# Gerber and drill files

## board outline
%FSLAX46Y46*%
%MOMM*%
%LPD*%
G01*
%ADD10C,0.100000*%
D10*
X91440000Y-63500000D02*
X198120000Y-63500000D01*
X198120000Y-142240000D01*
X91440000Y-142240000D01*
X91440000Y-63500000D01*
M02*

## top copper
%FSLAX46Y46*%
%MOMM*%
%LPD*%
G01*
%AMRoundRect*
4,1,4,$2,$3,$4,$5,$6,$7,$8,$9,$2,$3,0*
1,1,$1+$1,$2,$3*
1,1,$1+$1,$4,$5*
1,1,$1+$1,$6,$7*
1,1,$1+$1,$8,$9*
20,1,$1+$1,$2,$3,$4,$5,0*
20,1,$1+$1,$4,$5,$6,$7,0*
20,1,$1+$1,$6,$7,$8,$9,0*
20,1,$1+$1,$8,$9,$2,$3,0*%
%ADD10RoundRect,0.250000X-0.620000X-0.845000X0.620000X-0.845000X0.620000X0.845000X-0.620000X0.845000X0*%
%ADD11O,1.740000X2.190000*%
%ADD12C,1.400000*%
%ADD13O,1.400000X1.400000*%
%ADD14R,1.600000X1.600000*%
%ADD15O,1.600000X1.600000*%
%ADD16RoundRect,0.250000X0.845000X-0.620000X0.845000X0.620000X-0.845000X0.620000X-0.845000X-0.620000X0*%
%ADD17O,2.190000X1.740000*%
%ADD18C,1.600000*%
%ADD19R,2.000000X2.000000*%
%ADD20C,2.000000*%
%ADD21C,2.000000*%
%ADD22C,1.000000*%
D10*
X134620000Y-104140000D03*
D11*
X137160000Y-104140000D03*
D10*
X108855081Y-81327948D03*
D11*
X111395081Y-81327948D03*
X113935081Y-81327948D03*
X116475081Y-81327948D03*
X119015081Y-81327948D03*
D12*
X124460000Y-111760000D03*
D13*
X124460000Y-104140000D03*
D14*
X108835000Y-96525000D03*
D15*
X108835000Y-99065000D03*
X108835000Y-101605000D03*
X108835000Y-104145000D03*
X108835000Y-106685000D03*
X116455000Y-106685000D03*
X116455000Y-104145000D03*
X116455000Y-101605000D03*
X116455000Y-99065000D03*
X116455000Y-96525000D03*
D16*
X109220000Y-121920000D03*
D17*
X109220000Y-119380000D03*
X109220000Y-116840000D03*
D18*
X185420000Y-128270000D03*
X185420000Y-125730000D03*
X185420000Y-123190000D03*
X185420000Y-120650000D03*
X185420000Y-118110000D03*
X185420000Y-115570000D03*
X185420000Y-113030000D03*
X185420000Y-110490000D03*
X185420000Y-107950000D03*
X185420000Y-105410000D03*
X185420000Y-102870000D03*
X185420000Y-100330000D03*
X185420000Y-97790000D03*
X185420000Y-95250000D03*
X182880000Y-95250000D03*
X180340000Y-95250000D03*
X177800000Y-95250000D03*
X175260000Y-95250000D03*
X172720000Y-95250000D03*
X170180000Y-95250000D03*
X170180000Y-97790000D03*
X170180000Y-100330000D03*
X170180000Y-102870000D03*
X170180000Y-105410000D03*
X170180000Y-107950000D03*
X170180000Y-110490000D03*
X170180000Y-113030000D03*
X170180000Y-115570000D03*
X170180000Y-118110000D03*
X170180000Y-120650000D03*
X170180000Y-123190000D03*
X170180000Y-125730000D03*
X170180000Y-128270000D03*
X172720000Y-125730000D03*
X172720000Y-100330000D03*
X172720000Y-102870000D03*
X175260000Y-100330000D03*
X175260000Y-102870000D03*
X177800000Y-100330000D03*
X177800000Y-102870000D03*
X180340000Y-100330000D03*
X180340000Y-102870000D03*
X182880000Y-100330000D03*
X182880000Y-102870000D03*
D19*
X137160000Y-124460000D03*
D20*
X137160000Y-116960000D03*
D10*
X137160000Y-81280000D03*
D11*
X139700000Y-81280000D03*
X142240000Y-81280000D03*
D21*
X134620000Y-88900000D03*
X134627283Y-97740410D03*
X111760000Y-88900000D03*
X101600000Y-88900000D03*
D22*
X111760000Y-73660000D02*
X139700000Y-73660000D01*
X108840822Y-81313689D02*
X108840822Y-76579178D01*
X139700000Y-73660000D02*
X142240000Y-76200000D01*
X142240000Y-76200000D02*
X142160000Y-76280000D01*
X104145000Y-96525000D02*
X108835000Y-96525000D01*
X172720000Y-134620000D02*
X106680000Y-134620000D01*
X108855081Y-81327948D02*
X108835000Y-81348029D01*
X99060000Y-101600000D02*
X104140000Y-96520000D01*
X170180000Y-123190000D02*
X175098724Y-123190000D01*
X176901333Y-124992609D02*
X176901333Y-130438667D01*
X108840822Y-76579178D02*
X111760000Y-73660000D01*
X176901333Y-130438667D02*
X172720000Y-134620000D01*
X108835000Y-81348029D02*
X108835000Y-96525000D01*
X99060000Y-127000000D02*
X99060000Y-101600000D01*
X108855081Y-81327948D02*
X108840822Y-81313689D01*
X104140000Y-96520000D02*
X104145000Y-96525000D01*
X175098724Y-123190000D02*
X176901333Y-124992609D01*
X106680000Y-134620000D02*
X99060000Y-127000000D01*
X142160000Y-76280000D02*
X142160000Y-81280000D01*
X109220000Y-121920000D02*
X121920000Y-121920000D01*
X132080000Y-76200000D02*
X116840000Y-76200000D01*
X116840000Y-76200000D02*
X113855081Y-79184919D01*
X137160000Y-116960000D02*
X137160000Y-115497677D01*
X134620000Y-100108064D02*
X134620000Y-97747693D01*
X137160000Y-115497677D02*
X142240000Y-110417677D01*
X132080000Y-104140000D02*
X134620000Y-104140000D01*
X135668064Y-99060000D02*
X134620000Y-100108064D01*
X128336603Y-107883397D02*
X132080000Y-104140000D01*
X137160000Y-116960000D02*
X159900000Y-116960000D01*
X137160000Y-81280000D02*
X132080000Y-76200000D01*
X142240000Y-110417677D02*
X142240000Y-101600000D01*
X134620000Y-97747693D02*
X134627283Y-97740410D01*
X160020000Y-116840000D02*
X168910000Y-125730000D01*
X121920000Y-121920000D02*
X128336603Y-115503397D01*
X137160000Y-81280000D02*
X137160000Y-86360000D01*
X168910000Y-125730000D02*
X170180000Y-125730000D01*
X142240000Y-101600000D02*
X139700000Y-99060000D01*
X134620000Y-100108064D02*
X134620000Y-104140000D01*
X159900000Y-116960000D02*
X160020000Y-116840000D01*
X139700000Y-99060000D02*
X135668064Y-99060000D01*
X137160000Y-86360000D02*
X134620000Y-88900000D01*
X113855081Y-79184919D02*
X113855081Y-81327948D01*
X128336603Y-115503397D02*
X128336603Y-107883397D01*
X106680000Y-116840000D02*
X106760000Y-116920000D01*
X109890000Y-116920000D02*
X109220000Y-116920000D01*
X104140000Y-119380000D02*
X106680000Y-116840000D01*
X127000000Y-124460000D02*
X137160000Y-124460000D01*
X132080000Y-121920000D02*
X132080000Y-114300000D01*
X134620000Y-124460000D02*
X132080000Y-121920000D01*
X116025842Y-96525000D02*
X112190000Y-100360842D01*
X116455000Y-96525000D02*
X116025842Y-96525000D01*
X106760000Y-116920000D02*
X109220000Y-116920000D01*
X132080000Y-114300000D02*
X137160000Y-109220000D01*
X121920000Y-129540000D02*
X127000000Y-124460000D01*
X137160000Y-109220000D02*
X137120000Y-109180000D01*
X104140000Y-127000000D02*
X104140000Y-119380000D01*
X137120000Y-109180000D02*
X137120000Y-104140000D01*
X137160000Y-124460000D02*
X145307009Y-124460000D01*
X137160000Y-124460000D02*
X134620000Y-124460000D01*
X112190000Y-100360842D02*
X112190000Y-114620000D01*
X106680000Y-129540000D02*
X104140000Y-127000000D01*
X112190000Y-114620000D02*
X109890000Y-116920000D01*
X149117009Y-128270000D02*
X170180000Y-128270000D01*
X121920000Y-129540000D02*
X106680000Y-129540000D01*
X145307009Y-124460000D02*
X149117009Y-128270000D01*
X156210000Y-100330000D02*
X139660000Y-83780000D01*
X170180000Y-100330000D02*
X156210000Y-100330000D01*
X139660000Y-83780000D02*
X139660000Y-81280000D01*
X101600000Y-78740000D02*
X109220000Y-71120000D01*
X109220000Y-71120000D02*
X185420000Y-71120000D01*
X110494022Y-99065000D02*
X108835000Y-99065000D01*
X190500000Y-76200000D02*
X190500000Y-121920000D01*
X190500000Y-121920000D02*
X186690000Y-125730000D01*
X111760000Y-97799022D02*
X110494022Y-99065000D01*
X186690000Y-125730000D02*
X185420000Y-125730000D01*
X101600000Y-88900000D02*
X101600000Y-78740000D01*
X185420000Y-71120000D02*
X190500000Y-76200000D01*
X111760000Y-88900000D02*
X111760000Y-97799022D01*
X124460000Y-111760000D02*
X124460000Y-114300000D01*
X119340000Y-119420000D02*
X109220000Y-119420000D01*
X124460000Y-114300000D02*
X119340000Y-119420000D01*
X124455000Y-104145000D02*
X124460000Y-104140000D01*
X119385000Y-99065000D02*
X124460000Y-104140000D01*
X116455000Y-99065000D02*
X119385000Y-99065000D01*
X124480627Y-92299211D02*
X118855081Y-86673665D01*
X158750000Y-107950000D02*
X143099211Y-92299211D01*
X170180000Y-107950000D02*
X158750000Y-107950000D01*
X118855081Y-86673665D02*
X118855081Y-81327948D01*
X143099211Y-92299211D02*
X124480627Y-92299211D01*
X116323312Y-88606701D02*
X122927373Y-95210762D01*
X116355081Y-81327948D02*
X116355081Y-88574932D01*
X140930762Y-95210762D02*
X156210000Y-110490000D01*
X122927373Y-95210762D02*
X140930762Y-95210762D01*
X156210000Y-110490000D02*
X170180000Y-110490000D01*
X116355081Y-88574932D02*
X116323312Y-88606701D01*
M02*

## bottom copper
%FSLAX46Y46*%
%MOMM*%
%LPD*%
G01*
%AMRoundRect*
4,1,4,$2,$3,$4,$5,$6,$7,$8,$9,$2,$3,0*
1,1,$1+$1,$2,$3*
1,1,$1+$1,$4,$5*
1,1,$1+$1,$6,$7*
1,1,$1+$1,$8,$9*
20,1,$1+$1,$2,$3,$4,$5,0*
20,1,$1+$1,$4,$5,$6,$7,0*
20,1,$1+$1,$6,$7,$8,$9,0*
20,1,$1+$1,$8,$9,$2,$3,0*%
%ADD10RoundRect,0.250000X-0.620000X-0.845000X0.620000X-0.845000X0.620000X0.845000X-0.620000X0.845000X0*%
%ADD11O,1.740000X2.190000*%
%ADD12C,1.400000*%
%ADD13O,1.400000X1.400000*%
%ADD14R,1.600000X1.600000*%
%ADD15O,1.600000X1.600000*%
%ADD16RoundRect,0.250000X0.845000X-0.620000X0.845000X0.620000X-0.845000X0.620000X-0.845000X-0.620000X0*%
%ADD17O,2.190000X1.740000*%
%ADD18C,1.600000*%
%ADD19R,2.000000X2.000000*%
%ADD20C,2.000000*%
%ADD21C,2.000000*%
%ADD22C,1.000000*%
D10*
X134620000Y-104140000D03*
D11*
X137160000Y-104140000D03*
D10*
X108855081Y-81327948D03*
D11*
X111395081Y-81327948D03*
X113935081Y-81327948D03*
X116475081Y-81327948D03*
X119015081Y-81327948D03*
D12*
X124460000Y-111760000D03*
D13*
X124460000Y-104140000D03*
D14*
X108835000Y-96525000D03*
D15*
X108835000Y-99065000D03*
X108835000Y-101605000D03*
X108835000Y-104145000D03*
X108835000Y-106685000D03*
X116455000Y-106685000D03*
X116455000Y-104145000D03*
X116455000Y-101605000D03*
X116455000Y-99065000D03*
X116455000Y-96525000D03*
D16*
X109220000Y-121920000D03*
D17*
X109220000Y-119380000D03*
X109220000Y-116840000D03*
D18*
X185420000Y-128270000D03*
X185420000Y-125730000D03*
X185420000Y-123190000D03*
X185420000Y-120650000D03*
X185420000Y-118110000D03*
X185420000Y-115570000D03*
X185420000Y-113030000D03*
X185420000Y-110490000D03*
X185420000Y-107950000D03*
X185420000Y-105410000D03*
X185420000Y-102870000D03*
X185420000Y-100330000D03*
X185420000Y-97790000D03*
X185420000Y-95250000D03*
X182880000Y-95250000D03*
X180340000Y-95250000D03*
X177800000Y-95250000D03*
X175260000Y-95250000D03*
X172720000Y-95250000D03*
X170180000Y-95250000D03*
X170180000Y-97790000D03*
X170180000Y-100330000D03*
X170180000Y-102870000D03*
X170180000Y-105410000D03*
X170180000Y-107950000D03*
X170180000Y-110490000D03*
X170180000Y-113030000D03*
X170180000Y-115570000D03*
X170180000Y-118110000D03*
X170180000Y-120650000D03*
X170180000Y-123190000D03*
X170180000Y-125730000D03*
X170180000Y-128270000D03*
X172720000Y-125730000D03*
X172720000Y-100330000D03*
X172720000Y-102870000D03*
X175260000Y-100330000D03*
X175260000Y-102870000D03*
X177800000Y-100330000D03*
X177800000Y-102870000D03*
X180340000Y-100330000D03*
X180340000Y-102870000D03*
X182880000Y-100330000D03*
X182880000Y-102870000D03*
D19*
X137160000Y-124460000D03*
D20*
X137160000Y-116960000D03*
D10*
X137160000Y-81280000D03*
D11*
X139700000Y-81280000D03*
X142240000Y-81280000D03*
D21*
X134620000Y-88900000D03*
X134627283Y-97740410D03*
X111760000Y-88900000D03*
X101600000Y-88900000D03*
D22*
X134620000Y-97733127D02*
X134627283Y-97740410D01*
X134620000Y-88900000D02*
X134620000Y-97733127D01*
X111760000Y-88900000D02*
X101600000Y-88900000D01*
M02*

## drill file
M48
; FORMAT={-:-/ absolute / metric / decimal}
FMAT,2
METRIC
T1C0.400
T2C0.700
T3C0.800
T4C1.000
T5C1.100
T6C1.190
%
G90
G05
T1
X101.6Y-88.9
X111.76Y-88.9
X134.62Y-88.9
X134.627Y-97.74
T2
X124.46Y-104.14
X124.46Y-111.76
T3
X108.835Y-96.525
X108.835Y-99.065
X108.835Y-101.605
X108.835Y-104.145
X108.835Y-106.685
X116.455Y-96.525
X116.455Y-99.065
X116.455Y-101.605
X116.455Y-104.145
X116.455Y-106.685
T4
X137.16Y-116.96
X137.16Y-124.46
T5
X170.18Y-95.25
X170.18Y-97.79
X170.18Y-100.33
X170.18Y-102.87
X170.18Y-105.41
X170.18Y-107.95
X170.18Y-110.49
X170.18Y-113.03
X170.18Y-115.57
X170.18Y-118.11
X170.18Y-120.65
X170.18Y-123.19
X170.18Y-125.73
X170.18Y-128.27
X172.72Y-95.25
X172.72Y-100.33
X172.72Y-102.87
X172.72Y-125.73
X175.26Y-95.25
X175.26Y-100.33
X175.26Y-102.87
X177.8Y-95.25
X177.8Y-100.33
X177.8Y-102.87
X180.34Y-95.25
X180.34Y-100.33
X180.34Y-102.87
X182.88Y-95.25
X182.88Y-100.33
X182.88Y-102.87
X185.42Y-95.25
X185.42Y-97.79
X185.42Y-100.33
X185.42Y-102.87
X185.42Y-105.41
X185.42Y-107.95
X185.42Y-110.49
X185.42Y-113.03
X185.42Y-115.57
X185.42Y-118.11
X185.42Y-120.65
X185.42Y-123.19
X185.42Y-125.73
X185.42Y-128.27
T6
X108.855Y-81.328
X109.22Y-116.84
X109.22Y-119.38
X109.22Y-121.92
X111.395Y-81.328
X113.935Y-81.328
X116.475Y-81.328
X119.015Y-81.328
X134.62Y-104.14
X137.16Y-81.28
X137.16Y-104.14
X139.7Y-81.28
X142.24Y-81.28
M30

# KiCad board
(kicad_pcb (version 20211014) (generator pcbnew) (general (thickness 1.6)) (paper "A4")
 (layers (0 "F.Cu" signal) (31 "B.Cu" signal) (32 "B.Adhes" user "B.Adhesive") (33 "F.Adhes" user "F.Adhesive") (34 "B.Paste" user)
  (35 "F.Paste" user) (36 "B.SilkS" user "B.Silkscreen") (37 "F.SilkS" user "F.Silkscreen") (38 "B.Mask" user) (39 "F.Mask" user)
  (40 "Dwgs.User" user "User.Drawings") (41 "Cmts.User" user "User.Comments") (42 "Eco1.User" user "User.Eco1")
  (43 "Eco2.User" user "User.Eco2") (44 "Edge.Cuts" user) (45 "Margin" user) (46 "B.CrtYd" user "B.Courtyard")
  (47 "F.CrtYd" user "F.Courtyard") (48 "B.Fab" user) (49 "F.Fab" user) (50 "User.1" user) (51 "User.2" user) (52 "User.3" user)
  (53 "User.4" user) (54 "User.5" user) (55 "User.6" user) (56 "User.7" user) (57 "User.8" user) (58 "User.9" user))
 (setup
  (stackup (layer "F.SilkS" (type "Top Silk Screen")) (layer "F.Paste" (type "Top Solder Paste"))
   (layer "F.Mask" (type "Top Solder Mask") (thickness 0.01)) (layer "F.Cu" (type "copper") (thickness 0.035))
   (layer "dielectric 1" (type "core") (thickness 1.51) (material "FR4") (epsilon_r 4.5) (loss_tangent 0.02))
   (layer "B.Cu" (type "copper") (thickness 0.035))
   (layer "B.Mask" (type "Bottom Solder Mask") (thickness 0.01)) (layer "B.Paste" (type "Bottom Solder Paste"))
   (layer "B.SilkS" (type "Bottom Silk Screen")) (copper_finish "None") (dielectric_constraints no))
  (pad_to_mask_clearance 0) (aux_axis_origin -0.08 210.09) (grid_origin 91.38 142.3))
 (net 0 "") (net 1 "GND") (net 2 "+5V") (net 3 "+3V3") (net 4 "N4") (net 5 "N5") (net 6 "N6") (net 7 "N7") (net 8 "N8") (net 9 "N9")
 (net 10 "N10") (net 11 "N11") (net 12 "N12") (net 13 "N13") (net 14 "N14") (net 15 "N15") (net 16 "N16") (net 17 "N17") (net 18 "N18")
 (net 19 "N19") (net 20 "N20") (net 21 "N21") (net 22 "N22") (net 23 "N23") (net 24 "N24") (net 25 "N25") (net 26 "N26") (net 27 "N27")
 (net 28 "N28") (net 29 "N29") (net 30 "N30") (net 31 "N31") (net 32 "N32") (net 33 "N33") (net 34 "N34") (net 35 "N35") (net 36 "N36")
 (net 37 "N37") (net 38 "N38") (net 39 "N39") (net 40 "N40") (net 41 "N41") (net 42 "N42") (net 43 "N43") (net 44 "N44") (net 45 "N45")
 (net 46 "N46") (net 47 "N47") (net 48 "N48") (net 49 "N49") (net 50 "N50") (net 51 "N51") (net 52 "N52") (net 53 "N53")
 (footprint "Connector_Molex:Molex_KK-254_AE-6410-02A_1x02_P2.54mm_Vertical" (layer "F.Cu") (at 134.62 104.14)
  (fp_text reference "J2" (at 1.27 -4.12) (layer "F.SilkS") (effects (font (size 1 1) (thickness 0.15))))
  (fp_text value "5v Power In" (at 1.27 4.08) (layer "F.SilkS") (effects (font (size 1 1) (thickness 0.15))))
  (pad "1" thru_hole roundrect (at 0 0) (size 1.74 2.19) (drill 1.19) (layers *.Cu *.Mask) (roundrect_rratio 0.1436781609) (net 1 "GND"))
  (pad "2" thru_hole oval (at 2.54 0) (size 1.74 2.19) (drill 1.19) (layers *.Cu *.Mask) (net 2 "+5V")))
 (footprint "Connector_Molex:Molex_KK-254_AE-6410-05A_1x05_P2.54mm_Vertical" (layer "F.Cu") (at 108.855081 81.327948)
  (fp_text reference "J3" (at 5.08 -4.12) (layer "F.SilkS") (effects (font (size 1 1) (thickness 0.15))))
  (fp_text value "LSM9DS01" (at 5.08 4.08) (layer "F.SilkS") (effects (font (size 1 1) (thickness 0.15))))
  (pad "1" thru_hole roundrect (at 0 0) (size 1.74 2.19) (drill 1.19) (layers *.Cu *.Mask) (roundrect_rratio 0.1436781609) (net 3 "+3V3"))
  (pad "2" thru_hole oval (at 2.54 0) (size 1.74 2.19) (drill 1.19) (layers *.Cu *.Mask) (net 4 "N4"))
  (pad "3" thru_hole oval (at 5.08 0) (size 1.74 2.19) (drill 1.19) (layers *.Cu *.Mask) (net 1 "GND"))
  (pad "4" thru_hole oval (at 7.62 0) (size 1.74 2.19) (drill 1.19) (layers *.Cu *.Mask) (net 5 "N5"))
  (pad "5" thru_hole oval (at 10.16 0) (size 1.74 2.19) (drill 1.19) (layers *.Cu *.Mask) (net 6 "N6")))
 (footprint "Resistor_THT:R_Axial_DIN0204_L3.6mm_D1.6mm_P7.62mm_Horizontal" (layer "F.Cu") (at 124.46 111.76 90)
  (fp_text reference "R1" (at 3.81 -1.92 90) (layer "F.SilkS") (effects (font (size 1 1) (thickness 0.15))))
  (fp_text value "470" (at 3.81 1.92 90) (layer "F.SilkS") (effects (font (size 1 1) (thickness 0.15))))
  (pad "1" thru_hole circle (at 0 0 90) (size 1.4 1.4) (drill 0.7) (layers *.Cu *.Mask) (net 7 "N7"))
  (pad "2" thru_hole oval (at 7.62 0 90) (size 1.4 1.4) (drill 0.7) (layers *.Cu *.Mask) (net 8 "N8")))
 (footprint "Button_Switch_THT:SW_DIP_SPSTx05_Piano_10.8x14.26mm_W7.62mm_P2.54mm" (layer "F.Cu") (at 108.835 96.525)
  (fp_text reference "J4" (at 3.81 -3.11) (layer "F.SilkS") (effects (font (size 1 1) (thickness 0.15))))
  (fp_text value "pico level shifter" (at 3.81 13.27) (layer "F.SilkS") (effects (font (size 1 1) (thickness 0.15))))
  (pad "1" thru_hole rect (at 0 0) (size 1.6 1.6) (drill 0.8) (layers *.Cu *.Mask) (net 3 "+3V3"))
  (pad "2" thru_hole oval (at 0 2.54) (size 1.6 1.6) (drill 0.8) (layers *.Cu *.Mask) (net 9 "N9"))
  (pad "3" thru_hole oval (at 0 5.08) (size 1.6 1.6) (drill 0.8) (layers *.Cu *.Mask) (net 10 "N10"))
  (pad "4" thru_hole oval (at 0 7.62) (size 1.6 1.6) (drill 0.8) (layers *.Cu *.Mask) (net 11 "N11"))
  (pad "5" thru_hole oval (at 0 10.16) (size 1.6 1.6) (drill 0.8) (layers *.Cu *.Mask) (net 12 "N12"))
  (pad "6" thru_hole oval (at 7.62 10.16) (size 1.6 1.6) (drill 0.8) (layers *.Cu *.Mask) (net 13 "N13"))
  (pad "7" thru_hole oval (at 7.62 7.62) (size 1.6 1.6) (drill 0.8) (layers *.Cu *.Mask) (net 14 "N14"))
  (pad "8" thru_hole oval (at 7.62 5.08) (size 1.6 1.6) (drill 0.8) (layers *.Cu *.Mask) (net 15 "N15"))
  (pad "9" thru_hole oval (at 7.62 2.54) (size 1.6 1.6) (drill 0.8) (layers *.Cu *.Mask) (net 8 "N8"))
  (pad "10" thru_hole oval (at 7.62 0) (size 1.6 1.6) (drill 0.8) (layers *.Cu *.Mask) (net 2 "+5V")))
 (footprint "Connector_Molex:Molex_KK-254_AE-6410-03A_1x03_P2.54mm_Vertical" (layer "F.Cu") (at 109.22 121.92 90)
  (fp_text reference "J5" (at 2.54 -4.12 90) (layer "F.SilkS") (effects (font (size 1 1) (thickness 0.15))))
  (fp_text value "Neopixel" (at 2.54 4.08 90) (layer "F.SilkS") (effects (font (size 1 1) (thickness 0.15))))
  (pad "1" thru_hole roundrect (at 0 0 90) (size 1.74 2.19) (drill 1.19) (layers *.Cu *.Mask) (roundrect_rratio 0.1436781609) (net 1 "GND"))
  (pad "2" thru_hole oval (at 2.54 0 90) (size 1.74 2.19) (drill 1.19) (layers *.Cu *.Mask) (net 7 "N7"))
  (pad "3" thru_hole oval (at 5.08 0 90) (size 1.74 2.19) (drill 1.19) (layers *.Cu *.Mask) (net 2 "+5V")))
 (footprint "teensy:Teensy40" (layer "F.Cu") (at 177.8 111.76 90)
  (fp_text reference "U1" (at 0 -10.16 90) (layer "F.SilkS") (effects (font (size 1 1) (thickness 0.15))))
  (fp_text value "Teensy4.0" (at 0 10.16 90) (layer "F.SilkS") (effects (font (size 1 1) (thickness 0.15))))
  (pad "1" thru_hole circle locked (at -16.51 7.62 90) (size 1.6 1.6) (drill 1.1) (layers *.Cu *.Mask) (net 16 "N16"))
  (pad "2" thru_hole circle locked (at -13.97 7.62 90) (size 1.6 1.6) (drill 1.1) (layers *.Cu *.Mask) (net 9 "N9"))
  (pad "3" thru_hole circle locked (at -11.43 7.62 90) (size 1.6 1.6) (drill 1.1) (layers *.Cu *.Mask) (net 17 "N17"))
  (pad "4" thru_hole circle locked (at -8.89 7.62 90) (size 1.6 1.6) (drill 1.1) (layers *.Cu *.Mask) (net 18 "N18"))
  (pad "5" thru_hole circle locked (at -6.35 7.62 90) (size 1.6 1.6) (drill 1.1) (layers *.Cu *.Mask) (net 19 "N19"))
  (pad "6" thru_hole circle locked (at -3.81 7.62 90) (size 1.6 1.6) (drill 1.1) (layers *.Cu *.Mask) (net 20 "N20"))
  (pad "7" thru_hole circle locked (at -1.27 7.62 90) (size 1.6 1.6) (drill 1.1) (layers *.Cu *.Mask) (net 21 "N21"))
  (pad "8" thru_hole circle locked (at 1.27 7.62 90) (size 1.6 1.6) (drill 1.1) (layers *.Cu *.Mask) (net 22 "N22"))
  (pad "9" thru_hole circle locked (at 3.81 7.62 90) (size 1.6 1.6) (drill 1.1) (layers *.Cu *.Mask) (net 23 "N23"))
  (pad "10" thru_hole circle locked (at 6.35 7.62 90) (size 1.6 1.6) (drill 1.1) (layers *.Cu *.Mask) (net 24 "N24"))
  (pad "11" thru_hole circle locked (at 8.89 7.62 90) (size 1.6 1.6) (drill 1.1) (layers *.Cu *.Mask) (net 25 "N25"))
  (pad "12" thru_hole circle locked (at 11.43 7.62 90) (size 1.6 1.6) (drill 1.1) (layers *.Cu *.Mask) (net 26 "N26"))
  (pad "13" thru_hole circle locked (at 13.97 7.62 90) (size 1.6 1.6) (drill 1.1) (layers *.Cu *.Mask) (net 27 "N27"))
  (pad "14" thru_hole circle locked (at 16.51 7.62 90) (size 1.6 1.6) (drill 1.1) (layers *.Cu *.Mask) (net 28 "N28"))
  (pad "15" thru_hole circle locked (at 16.51 5.08 90) (size 1.6 1.6) (drill 1.1) (layers *.Cu *.Mask) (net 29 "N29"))
  (pad "16" thru_hole circle locked (at 16.51 2.54 90) (size 1.6 1.6) (drill 1.1) (layers *.Cu *.Mask) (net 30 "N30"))
  (pad "17" thru_hole circle locked (at 16.51 0 90) (size 1.6 1.6) (drill 1.1) (layers *.Cu *.Mask) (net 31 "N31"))
  (pad "18" thru_hole circle locked (at 16.51 -2.54 90) (size 1.6 1.6) (drill 1.1) (layers *.Cu *.Mask) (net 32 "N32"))
  (pad "19" thru_hole circle locked (at 16.51 -5.08 90) (size 1.6 1.6) (drill 1.1) (layers *.Cu *.Mask) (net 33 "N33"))
  (pad "20" thru_hole circle locked (at 16.51 -7.62 90) (size 1.6 1.6) (drill 1.1) (layers *.Cu *.Mask) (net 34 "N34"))
  (pad "21" thru_hole circle locked (at 13.97 -7.62 90) (size 1.6 1.6) (drill 1.1) (layers *.Cu *.Mask) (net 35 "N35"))
  (pad "22" thru_hole circle locked (at 11.43 -7.62 90) (size 1.6 1.6) (drill 1.1) (layers *.Cu *.Mask) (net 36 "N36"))
  (pad "23" thru_hole circle locked (at 8.89 -7.62 90) (size 1.6 1.6) (drill 1.1) (layers *.Cu *.Mask) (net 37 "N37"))
  (pad "24" thru_hole circle locked (at 6.35 -7.62 90) (size 1.6 1.6) (drill 1.1) (layers *.Cu *.Mask) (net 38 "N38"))
  (pad "25" thru_hole circle locked (at 3.81 -7.62 90) (size 1.6 1.6) (drill 1.1) (layers *.Cu *.Mask) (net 6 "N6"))
  (pad "26" thru_hole circle locked (at 1.27 -7.62 90) (size 1.6 1.6) (drill 1.1) (layers *.Cu *.Mask) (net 5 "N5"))
  (pad "27" thru_hole circle locked (at -1.27 -7.62 90) (size 1.6 1.6) (drill 1.1) (layers *.Cu *.Mask) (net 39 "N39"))
  (pad "28" thru_hole circle locked (at -3.81 -7.62 90) (size 1.6 1.6) (drill 1.1) (layers *.Cu *.Mask) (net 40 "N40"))
  (pad "29" thru_hole circle locked (at -6.35 -7.62 90) (size 1.6 1.6) (drill 1.1) (layers *.Cu *.Mask) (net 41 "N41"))
  (pad "30" thru_hole circle locked (at -8.89 -7.62 90) (size 1.6 1.6) (drill 1.1) (layers *.Cu *.Mask) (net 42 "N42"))
  (pad "31" thru_hole circle locked (at -11.43 -7.62 90) (size 1.6 1.6) (drill 1.1) (layers *.Cu *.Mask) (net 3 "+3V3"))
  (pad "32" thru_hole circle locked (at -13.97 -7.62 90) (size 1.6 1.6) (drill 1.1) (layers *.Cu *.Mask) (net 1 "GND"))
  (pad "33" thru_hole circle locked (at -16.51 -7.62 90) (size 1.6 1.6) (drill 1.1) (layers *.Cu *.Mask) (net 2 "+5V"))
  (pad "34" thru_hole circle locked (at -13.97 -5.08 90) (size 1.6 1.6) (drill 1.1) (layers *.Cu *.Mask) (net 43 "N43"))
  (pad "35" thru_hole circle locked (at 11.43 -5.08 90) (size 1.6 1.6) (drill 1.1) (layers *.Cu *.Mask) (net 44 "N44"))
  (pad "36" thru_hole circle locked (at 8.89 -5.08 90) (size 1.6 1.6) (drill 1.1) (layers *.Cu *.Mask) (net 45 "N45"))
  (pad "37" thru_hole circle locked (at 11.43 -2.54 90) (size 1.6 1.6) (drill 1.1) (layers *.Cu *.Mask) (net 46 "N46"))
  (pad "38" thru_hole circle locked (at 8.89 -2.54 90) (size 1.6 1.6) (drill 1.1) (layers *.Cu *.Mask) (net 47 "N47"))
  (pad "39" thru_hole circle locked (at 11.43 0 90) (size 1.6 1.6) (drill 1.1) (layers *.Cu *.Mask) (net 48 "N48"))
  (pad "40" thru_hole circle locked (at 8.89 0 90) (size 1.6 1.6) (drill 1.1) (layers *.Cu *.Mask) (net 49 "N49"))
  (pad "41" thru_hole circle locked (at 11.43 2.54 90) (size 1.6 1.6) (drill 1.1) (layers *.Cu *.Mask) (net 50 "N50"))
  (pad "42" thru_hole circle locked (at 8.89 2.54 90) (size 1.6 1.6) (drill 1.1) (layers *.Cu *.Mask) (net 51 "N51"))
  (pad "43" thru_hole circle locked (at 11.43 5.08 90) (size 1.6 1.6) (drill 1.1) (layers *.Cu *.Mask) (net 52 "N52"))
  (pad "44" thru_hole circle locked (at 8.89 5.08 90) (size 1.6 1.6) (drill 1.1) (layers *.Cu *.Mask) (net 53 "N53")))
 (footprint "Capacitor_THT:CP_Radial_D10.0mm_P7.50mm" (layer "F.Cu") (at 137.16 124.46 90)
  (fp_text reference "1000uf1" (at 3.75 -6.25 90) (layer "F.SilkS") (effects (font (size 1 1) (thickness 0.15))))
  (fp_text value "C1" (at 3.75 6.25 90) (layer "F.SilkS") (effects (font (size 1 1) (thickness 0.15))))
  (pad "1" thru_hole rect (at 0 0 90) (size 2 2) (drill 1) (layers *.Cu *.Mask) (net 2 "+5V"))
  (pad "2" thru_hole circle (at 7.5 0 90) (size 2 2) (drill 1) (layers *.Cu *.Mask) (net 1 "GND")))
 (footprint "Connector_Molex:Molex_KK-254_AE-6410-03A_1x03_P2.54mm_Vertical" (layer "F.Cu") (at 137.16 81.28)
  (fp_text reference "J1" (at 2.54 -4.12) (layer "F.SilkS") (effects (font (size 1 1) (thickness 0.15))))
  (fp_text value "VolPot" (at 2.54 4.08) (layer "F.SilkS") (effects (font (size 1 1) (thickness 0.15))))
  (pad "1" thru_hole roundrect (at 0 0) (size 1.74 2.19) (drill 1.19) (layers *.Cu *.Mask) (roundrect_rratio 0.1436781609) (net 1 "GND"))
  (pad "2" thru_hole oval (at 2.54 0) (size 1.74 2.19) (drill 1.19) (layers *.Cu *.Mask) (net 36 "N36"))
  (pad "3" thru_hole oval (at 5.08 0) (size 1.74 2.19) (drill 1.19) (layers *.Cu *.Mask) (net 3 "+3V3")))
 (gr_rect (start 91.44 63.5) (end 198.12 142.24) (layer "Edge.Cuts") (width 0.1) (fill none))
 (segment (start 111.76 73.66) (end 139.7 73.66) (width 1) (layer "F.Cu") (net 3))
 (segment (start 108.840822 81.313689) (end 108.840822 76.579178) (width 1) (layer "F.Cu") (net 3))
 (segment (start 139.7 73.66) (end 142.24 76.2) (width 1) (layer "F.Cu") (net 3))
 (segment (start 142.24 76.2) (end 142.16 76.28) (width 1) (layer "F.Cu") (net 3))
 (segment (start 104.145 96.525) (end 108.835 96.525) (width 1) (layer "F.Cu") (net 3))
 (segment (start 172.72 134.62) (end 106.68 134.62) (width 1) (layer "F.Cu") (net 3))
 (segment (start 108.855081 81.327948) (end 108.835 81.348029) (width 1) (layer "F.Cu") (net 3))
 (segment (start 99.06 101.6) (end 104.14 96.52) (width 1) (layer "F.Cu") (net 3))
 (segment (start 170.18 123.19) (end 175.098724 123.19) (width 1) (layer "F.Cu") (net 3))
 (segment (start 176.901333 124.992609) (end 176.901333 130.438667) (width 1) (layer "F.Cu") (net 3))
 (segment (start 108.840822 76.579178) (end 111.76 73.66) (width 1) (layer "F.Cu") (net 3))
 (segment (start 176.901333 130.438667) (end 172.72 134.62) (width 1) (layer "F.Cu") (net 3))
 (segment (start 108.835 81.348029) (end 108.835 96.525) (width 1) (layer "F.Cu") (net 3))
 (segment (start 99.06 127) (end 99.06 101.6) (width 1) (layer "F.Cu") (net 3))
 (segment (start 108.855081 81.327948) (end 108.840822 81.313689) (width 1) (layer "F.Cu") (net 3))
 (segment (start 104.14 96.52) (end 104.145 96.525) (width 1) (layer "F.Cu") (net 3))
 (segment (start 175.098724 123.19) (end 176.901333 124.992609) (width 1) (layer "F.Cu") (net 3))
 (segment (start 106.68 134.62) (end 99.06 127) (width 1) (layer "F.Cu") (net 3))
 (segment (start 142.16 76.28) (end 142.16 81.28) (width 1) (layer "F.Cu") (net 3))
 (segment (start 109.22 121.92) (end 121.92 121.92) (width 1) (layer "F.Cu") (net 1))
 (segment (start 132.08 76.2) (end 116.84 76.2) (width 1) (layer "F.Cu") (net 1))
 (segment (start 116.84 76.2) (end 113.855081 79.184919) (width 1) (layer "F.Cu") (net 1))
 (segment (start 137.16 116.96) (end 137.16 115.497677) (width 1) (layer "F.Cu") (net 1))
 (segment (start 134.62 100.108064) (end 134.62 97.747693) (width 1) (layer "F.Cu") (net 1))
 (segment (start 137.16 115.497677) (end 142.24 110.417677) (width 1) (layer "F.Cu") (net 1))
 (segment (start 132.08 104.14) (end 134.62 104.14) (width 1) (layer "F.Cu") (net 1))
 (segment (start 135.668064 99.06) (end 134.62 100.108064) (width 1) (layer "F.Cu") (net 1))
 (segment (start 128.336603 107.883397) (end 132.08 104.14) (width 1) (layer "F.Cu") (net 1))
 (segment (start 137.16 116.96) (end 159.9 116.96) (width 1) (layer "F.Cu") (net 1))
 (segment (start 137.16 81.28) (end 132.08 76.2) (width 1) (layer "F.Cu") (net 1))
 (segment (start 142.24 110.417677) (end 142.24 101.6) (width 1) (layer "F.Cu") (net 1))
 (segment (start 134.62 97.747693) (end 134.627283 97.74041) (width 1) (layer "F.Cu") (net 1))
 (segment (start 160.02 116.84) (end 168.91 125.73) (width 1) (layer "F.Cu") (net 1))
 (segment (start 121.92 121.92) (end 128.336603 115.503397) (width 1) (layer "F.Cu") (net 1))
 (segment (start 137.16 81.28) (end 137.16 86.36) (width 1) (layer "F.Cu") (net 1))
 (segment (start 168.91 125.73) (end 170.18 125.73) (width 1) (layer "F.Cu") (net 1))
 (segment (start 142.24 101.6) (end 139.7 99.06) (width 1) (layer "F.Cu") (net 1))
 (segment (start 134.62 100.108064) (end 134.62 104.14) (width 1) (layer "F.Cu") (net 1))
 (segment (start 159.9 116.96) (end 160.02 116.84) (width 1) (layer "F.Cu") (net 1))
 (segment (start 139.7 99.06) (end 135.668064 99.06) (width 1) (layer "F.Cu") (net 1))
 (segment (start 137.16 86.36) (end 134.62 88.9) (width 1) (layer "F.Cu") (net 1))
 (segment (start 113.855081 79.184919) (end 113.855081 81.327948) (width 1) (layer "F.Cu") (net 1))
 (segment (start 128.336603 115.503397) (end 128.336603 107.883397) (width 1) (layer "F.Cu") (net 1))
 (via (at 134.62 88.9) (size 2) (drill 0.4) (layers "F.Cu" "B.Cu") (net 1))
 (via (at 134.627283 97.74041) (size 2) (drill 0.4) (layers "F.Cu" "B.Cu") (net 1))
 (segment (start 134.62 97.733127) (end 134.627283 97.74041) (width 1) (layer "B.Cu") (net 1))
 (segment (start 134.62 88.9) (end 134.62 97.733127) (width 1) (layer "B.Cu") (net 1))
 (segment (start 106.68 116.84) (end 106.76 116.92) (width 1) (layer "F.Cu") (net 2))
 (segment (start 109.89 116.92) (end 109.22 116.92) (width 1) (layer "F.Cu") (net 2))
 (segment (start 104.14 119.38) (end 106.68 116.84) (width 1) (layer "F.Cu") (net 2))
 (segment (start 127 124.46) (end 137.16 124.46) (width 1) (layer "F.Cu") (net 2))
 (segment (start 132.08 121.92) (end 132.08 114.3) (width 1) (layer "F.Cu") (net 2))
 (segment (start 134.62 124.46) (end 132.08 121.92) (width 1) (layer "F.Cu") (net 2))
 (segment (start 116.025842 96.525) (end 112.19 100.360842) (width 1) (layer "F.Cu") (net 2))
 (segment (start 116.455 96.525) (end 116.025842 96.525) (width 1) (layer "F.Cu") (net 2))
 (segment (start 106.76 116.92) (end 109.22 116.92) (width 1) (layer "F.Cu") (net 2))
 (segment (start 132.08 114.3) (end 137.16 109.22) (width 1) (layer "F.Cu") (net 2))
 (segment (start 121.92 129.54) (end 127 124.46) (width 1) (layer "F.Cu") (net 2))
 (segment (start 137.16 109.22) (end 137.12 109.18) (width 1) (layer "F.Cu") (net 2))
 (segment (start 104.14 127) (end 104.14 119.38) (width 1) (layer "F.Cu") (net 2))
 (segment (start 137.12 109.18) (end 137.12 104.14) (width 1) (layer "F.Cu") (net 2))
 (segment (start 137.16 124.46) (end 145.307009 124.46) (width 1) (layer "F.Cu") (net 2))
 (segment (start 137.16 124.46) (end 134.62 124.46) (width 1) (layer "F.Cu") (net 2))
 (segment (start 112.19 100.360842) (end 112.19 114.62) (width 1) (layer "F.Cu") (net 2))
 (segment (start 106.68 129.54) (end 104.14 127) (width 1) (layer "F.Cu") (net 2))
 (segment (start 112.19 114.62) (end 109.89 116.92) (width 1) (layer "F.Cu") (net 2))
 (segment (start 149.117009 128.27) (end 170.18 128.27) (width 1) (layer "F.Cu") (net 2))
 (segment (start 121.92 129.54) (end 106.68 129.54) (width 1) (layer "F.Cu") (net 2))
 (segment (start 145.307009 124.46) (end 149.117009 128.27) (width 1) (layer "F.Cu") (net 2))
 (segment (start 156.21 100.33) (end 139.66 83.78) (width 1) (layer "F.Cu") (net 36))
 (segment (start 170.18 100.33) (end 156.21 100.33) (width 1) (layer "F.Cu") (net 36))
 (segment (start 139.66 83.78) (end 139.66 81.28) (width 1) (layer "F.Cu") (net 36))
 (segment (start 101.6 78.74) (end 109.22 71.12) (width 1) (layer "F.Cu") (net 9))
 (segment (start 109.22 71.12) (end 185.42 71.12) (width 1) (layer "F.Cu") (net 9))
 (segment (start 110.494022 99.065) (end 108.835 99.065) (width 1) (layer "F.Cu") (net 9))
 (segment (start 190.5 76.2) (end 190.5 121.92) (width 1) (layer "F.Cu") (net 9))
 (segment (start 190.5 121.92) (end 186.69 125.73) (width 1) (layer "F.Cu") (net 9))
 (segment (start 111.76 97.799022) (end 110.494022 99.065) (width 1) (layer "F.Cu") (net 9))
 (segment (start 186.69 125.73) (end 185.42 125.73) (width 1) (layer "F.Cu") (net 9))
 (segment (start 101.6 88.9) (end 101.6 78.74) (width 1) (layer "F.Cu") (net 9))
 (segment (start 185.42 71.12) (end 190.5 76.2) (width 1) (layer "F.Cu") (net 9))
 (segment (start 111.76 88.9) (end 111.76 97.799022) (width 1) (layer "F.Cu") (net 9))
 (via (at 111.76 88.9) (size 2) (drill 0.4) (layers "F.Cu" "B.Cu") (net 9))
 (via (at 101.6 88.9) (size 2) (drill 0.4) (layers "F.Cu" "B.Cu") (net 9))
 (segment (start 111.76 88.9) (end 101.6 88.9) (width 1) (layer "B.Cu") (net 9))
 (segment (start 124.46 111.76) (end 124.46 114.3) (width 1) (layer "F.Cu") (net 7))
 (segment (start 119.34 119.42) (end 109.22 119.42) (width 1) (layer "F.Cu") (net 7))
 (segment (start 124.46 114.3) (end 119.34 119.42) (width 1) (layer "F.Cu") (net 7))
 (segment (start 124.455 104.145) (end 124.46 104.14) (width 1) (layer "F.Cu") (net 8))
 (segment (start 119.385 99.065) (end 124.46 104.14) (width 1) (layer "F.Cu") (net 8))
 (segment (start 116.455 99.065) (end 119.385 99.065) (width 1) (layer "F.Cu") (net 8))
 (segment (start 124.480627 92.299211) (end 118.855081 86.673665) (width 1) (layer "F.Cu") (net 6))
 (segment (start 158.75 107.95) (end 143.099211 92.299211) (width 1) (layer "F.Cu") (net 6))
 (segment (start 170.18 107.95) (end 158.75 107.95) (width 1) (layer "F.Cu") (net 6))
 (segment (start 118.855081 86.673665) (end 118.855081 81.327948) (width 1) (layer "F.Cu") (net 6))
 (segment (start 143.099211 92.299211) (end 124.480627 92.299211) (width 1) (layer "F.Cu") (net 6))
 (segment (start 116.323312 88.606701) (end 122.927373 95.210762) (width 1) (layer "F.Cu") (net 5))
 (segment (start 116.355081 81.327948) (end 116.355081 88.574932) (width 1) (layer "F.Cu") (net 5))
 (segment (start 140.930762 95.210762) (end 156.21 110.49) (width 1) (layer "F.Cu") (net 5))
 (segment (start 122.927373 95.210762) (end 140.930762 95.210762) (width 1) (layer "F.Cu") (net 5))
 (segment (start 156.21 110.49) (end 170.18 110.49) (width 1) (layer "F.Cu") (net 5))
 (segment (start 116.355081 88.574932) (end 116.323312 88.606701) (width 1) (layer "F.Cu") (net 5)))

